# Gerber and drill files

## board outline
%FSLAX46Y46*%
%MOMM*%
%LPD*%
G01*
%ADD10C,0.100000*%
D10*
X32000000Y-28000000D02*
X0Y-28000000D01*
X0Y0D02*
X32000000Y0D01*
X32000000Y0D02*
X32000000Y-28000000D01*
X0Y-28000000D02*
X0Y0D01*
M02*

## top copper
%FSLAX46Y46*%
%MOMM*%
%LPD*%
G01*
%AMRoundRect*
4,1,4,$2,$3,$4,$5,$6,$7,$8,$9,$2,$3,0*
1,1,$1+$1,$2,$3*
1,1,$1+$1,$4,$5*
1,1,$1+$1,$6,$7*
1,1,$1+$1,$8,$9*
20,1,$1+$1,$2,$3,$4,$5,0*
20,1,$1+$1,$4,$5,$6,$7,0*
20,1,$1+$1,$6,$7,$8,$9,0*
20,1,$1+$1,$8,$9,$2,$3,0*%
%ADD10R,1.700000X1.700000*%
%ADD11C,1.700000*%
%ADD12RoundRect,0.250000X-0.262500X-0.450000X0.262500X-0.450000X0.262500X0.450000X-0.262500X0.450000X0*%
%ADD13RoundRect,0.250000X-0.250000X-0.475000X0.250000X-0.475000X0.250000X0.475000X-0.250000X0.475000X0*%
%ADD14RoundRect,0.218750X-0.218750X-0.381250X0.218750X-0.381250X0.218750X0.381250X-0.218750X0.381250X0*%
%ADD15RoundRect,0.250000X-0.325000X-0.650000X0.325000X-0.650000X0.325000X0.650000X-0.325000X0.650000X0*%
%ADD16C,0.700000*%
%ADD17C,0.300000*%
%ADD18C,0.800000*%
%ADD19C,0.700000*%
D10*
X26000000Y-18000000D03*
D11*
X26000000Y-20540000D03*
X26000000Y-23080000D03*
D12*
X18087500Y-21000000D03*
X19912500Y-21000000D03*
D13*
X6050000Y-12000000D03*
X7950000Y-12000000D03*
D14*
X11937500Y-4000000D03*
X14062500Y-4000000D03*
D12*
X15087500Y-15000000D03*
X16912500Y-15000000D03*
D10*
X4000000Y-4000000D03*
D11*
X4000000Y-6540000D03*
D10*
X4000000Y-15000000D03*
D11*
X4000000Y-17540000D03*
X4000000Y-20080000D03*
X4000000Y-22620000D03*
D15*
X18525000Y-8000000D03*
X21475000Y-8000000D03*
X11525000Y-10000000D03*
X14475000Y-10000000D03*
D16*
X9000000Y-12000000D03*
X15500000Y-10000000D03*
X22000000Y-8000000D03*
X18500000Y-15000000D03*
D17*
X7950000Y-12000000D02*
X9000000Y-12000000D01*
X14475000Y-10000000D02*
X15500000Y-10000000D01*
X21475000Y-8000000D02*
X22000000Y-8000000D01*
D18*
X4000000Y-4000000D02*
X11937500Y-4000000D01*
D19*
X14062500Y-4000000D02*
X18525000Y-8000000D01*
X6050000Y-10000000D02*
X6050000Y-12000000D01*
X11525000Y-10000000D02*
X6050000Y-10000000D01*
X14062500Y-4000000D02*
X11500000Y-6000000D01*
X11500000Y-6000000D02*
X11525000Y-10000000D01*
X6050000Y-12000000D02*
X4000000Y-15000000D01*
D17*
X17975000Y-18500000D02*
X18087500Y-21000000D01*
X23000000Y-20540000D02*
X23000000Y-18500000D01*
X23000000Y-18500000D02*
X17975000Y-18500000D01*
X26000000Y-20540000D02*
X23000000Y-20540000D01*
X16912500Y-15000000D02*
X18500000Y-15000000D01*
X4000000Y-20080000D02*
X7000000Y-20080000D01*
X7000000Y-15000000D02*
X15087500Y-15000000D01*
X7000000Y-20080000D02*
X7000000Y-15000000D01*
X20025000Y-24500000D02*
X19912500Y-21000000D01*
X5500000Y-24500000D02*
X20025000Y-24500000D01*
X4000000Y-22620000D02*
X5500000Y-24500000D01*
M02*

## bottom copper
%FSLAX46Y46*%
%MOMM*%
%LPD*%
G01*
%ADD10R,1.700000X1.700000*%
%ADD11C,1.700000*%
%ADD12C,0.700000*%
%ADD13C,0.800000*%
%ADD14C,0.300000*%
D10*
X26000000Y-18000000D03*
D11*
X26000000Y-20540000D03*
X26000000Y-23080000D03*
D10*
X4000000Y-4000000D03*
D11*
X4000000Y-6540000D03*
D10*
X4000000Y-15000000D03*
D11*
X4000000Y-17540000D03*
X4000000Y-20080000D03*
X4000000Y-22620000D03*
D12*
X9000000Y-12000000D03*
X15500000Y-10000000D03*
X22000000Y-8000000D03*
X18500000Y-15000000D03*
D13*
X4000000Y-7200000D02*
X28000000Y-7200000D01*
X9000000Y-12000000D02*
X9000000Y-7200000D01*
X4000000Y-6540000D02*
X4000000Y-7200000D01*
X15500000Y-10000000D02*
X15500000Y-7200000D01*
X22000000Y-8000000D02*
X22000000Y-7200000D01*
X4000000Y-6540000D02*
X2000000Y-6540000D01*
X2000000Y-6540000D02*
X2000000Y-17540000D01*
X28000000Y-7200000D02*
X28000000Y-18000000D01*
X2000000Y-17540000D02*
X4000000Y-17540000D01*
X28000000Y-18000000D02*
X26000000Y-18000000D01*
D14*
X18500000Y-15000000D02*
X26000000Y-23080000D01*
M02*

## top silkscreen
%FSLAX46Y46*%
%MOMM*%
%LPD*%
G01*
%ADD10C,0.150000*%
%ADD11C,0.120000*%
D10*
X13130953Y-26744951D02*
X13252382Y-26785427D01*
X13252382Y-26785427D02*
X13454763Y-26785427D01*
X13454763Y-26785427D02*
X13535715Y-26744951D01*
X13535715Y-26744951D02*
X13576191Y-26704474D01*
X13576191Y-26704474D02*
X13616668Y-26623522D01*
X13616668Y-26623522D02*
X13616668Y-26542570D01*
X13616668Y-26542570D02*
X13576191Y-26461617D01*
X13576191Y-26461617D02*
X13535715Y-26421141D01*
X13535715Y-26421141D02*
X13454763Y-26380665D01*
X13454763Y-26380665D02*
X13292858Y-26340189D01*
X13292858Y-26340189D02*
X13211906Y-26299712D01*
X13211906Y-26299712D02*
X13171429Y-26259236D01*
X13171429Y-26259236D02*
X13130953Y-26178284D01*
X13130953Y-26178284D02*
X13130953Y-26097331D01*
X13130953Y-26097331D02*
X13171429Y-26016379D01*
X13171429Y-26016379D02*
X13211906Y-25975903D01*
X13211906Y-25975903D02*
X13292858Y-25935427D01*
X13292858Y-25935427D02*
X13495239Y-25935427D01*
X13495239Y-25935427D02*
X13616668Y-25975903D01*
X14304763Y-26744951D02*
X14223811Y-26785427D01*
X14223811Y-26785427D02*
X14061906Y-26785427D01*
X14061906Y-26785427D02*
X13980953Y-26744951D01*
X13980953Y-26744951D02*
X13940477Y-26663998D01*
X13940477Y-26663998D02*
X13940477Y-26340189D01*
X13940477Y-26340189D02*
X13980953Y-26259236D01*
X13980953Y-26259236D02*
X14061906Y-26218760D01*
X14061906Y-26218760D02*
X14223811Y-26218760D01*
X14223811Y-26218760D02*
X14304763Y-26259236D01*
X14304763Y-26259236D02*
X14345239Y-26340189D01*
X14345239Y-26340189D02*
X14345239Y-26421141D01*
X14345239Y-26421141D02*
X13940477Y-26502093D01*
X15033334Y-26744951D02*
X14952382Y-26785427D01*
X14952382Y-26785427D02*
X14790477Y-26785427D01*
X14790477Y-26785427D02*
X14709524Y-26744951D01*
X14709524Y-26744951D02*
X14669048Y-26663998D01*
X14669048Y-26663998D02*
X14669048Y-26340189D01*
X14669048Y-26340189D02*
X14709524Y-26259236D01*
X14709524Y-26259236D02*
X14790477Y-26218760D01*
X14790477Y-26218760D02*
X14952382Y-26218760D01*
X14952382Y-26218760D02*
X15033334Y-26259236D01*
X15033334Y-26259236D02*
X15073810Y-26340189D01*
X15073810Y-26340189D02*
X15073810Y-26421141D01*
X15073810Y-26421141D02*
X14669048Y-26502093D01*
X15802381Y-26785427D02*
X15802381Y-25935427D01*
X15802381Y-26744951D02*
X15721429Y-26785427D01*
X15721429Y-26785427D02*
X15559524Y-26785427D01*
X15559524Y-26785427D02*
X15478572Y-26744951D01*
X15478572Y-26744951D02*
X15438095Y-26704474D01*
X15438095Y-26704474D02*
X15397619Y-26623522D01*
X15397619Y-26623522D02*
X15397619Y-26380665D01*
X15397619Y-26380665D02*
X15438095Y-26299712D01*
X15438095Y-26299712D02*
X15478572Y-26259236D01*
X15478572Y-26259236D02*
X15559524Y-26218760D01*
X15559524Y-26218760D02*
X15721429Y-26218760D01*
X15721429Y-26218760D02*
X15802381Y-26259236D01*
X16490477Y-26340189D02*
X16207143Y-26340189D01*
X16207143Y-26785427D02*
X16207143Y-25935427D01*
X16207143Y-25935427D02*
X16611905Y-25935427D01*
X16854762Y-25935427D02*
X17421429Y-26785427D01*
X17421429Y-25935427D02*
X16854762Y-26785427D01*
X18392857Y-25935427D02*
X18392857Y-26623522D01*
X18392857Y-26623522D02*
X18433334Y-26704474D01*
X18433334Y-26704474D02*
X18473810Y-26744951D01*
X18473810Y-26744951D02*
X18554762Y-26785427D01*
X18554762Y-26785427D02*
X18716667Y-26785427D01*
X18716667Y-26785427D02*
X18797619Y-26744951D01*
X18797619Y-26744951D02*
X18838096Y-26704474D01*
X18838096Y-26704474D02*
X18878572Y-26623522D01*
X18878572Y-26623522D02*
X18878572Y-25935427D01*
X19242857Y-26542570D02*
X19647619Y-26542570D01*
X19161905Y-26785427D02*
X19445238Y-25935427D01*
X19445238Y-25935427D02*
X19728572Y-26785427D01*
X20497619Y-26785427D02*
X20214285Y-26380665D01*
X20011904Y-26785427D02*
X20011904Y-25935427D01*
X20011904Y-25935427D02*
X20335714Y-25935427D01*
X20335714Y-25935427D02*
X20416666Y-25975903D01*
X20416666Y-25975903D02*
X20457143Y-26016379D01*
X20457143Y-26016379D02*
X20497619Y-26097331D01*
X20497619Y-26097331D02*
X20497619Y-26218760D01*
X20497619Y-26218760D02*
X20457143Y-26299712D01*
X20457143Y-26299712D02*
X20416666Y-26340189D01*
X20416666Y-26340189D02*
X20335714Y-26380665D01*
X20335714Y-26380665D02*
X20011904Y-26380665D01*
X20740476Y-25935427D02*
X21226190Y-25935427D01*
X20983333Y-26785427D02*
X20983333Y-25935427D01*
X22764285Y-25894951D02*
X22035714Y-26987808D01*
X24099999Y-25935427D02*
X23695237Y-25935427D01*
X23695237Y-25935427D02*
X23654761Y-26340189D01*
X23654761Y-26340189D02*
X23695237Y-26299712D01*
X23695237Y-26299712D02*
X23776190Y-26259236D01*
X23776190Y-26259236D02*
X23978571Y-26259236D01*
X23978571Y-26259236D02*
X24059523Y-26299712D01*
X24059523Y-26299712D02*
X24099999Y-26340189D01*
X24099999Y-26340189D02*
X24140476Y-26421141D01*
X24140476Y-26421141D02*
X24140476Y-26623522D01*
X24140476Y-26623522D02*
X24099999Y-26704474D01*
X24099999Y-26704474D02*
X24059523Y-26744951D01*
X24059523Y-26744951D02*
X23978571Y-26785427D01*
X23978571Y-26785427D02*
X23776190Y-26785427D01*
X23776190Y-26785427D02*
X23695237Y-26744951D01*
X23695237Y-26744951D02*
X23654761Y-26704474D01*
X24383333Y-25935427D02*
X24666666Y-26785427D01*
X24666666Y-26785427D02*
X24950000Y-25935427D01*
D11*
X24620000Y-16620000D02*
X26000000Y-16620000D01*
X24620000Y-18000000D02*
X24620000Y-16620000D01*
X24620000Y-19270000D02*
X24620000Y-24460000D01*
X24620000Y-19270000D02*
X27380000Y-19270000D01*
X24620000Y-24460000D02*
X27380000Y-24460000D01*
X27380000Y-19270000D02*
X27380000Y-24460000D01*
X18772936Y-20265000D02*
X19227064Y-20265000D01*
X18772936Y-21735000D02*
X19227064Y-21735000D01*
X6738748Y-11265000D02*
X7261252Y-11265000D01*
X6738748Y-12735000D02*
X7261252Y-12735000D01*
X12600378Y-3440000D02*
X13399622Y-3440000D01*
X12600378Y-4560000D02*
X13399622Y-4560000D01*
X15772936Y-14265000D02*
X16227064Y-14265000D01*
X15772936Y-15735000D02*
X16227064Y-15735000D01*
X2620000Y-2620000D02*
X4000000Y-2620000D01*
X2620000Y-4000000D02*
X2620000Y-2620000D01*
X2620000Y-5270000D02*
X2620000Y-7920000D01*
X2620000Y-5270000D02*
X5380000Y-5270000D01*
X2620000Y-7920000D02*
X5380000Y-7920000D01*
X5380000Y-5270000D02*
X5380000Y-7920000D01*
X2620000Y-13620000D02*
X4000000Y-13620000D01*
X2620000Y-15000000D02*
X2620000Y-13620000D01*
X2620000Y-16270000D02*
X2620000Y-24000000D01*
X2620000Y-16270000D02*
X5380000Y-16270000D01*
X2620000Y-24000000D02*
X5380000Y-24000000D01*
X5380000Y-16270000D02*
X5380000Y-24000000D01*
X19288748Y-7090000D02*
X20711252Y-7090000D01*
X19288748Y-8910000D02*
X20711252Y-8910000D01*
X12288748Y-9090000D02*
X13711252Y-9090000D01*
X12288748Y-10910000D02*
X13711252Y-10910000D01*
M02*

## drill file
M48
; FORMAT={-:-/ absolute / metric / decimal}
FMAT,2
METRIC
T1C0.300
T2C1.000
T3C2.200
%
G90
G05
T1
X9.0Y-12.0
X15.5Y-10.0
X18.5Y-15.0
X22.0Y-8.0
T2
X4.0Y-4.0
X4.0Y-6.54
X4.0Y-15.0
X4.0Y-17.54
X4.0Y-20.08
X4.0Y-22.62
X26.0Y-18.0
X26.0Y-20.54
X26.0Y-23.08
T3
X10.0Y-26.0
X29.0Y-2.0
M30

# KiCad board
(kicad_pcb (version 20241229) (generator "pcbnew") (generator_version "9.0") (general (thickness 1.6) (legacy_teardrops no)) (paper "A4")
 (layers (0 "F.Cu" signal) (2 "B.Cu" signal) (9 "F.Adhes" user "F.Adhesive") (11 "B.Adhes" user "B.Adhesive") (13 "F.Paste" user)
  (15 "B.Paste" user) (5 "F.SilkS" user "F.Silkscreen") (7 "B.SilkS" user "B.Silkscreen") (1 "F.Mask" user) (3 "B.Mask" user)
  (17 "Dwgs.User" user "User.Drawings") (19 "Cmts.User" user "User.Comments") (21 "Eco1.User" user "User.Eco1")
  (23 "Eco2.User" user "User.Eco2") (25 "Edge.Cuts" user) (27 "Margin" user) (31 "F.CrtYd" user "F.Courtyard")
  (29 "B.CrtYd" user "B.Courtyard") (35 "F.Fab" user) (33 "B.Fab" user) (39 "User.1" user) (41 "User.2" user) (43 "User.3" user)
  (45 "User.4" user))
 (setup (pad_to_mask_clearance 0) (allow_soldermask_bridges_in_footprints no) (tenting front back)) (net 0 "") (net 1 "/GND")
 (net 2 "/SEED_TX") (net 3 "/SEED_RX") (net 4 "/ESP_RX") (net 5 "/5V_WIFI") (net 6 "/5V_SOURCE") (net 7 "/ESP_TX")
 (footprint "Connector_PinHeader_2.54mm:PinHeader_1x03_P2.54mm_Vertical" (layer "F.Cu") (at 26 18)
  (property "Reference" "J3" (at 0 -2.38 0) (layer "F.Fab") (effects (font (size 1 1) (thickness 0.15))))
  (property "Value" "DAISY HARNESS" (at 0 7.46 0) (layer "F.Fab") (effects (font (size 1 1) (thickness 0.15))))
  (fp_line (start -1.38 -1.38) (end 0 -1.38) (stroke (width 0.12) (type solid)) (layer "F.SilkS"))
  (fp_line (start -1.38 0) (end -1.38 -1.38) (stroke (width 0.12) (type solid)) (layer "F.SilkS"))
  (fp_line (start -1.38 1.27) (end -1.38 6.46) (stroke (width 0.12) (type solid)) (layer "F.SilkS"))
  (fp_line (start -1.38 1.27) (end 1.38 1.27) (stroke (width 0.12) (type solid)) (layer "F.SilkS"))
  (fp_line (start -1.38 6.46) (end 1.38 6.46) (stroke (width 0.12) (type solid)) (layer "F.SilkS"))
  (fp_line (start 1.38 1.27) (end 1.38 6.46) (stroke (width 0.12) (type solid)) (layer "F.SilkS"))
  (pad "1" thru_hole rect (at 0 0) (size 1.7 1.7) (drill 1) (layers "*.Cu" "*.Mask") (remove_unused_layers no) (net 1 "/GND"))
  (pad "2" thru_hole circle (at 0 2.54) (size 1.7 1.7) (drill 1) (layers "*.Cu" "*.Mask") (remove_unused_layers no) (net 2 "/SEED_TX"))
  (pad "3" thru_hole circle (at 0 5.08) (size 1.7 1.7) (drill 1) (layers "*.Cu" "*.Mask") (remove_unused_layers no) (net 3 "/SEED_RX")))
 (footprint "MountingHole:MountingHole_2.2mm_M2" (layer "F.Cu") (at 10 26)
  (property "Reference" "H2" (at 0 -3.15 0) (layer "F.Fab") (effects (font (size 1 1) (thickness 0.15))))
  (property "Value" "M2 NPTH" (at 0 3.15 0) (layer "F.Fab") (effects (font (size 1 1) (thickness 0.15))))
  (pad "" np_thru_hole circle (at 0 0) (size 2.2 2.2) (drill 2.2) (layers "*.Cu" "*.Mask")))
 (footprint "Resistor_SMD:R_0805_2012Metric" (layer "F.Cu") (at 19 21)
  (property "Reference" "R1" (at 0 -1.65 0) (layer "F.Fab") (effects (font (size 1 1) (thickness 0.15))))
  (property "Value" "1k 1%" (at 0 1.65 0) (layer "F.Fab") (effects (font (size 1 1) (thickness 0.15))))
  (fp_line (start -0.227064 -0.735) (end 0.227064 -0.735) (stroke (width 0.12) (type solid)) (layer "F.SilkS"))
  (fp_line (start -0.227064 0.735) (end 0.227064 0.735) (stroke (width 0.12) (type solid)) (layer "F.SilkS"))
  (pad "1" smd roundrect (at -0.9125 0) (size 1.025 1.4) (layers "F.Cu" "F.Mask" "F.Paste") (roundrect_rratio 0.243902) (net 2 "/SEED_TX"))
  (pad "2" smd roundrect (at 0.9125 0) (size 1.025 1.4) (layers "F.Cu" "F.Mask" "F.Paste") (roundrect_rratio 0.243902) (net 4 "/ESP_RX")))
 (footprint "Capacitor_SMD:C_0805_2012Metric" (layer "F.Cu") (at 7 12)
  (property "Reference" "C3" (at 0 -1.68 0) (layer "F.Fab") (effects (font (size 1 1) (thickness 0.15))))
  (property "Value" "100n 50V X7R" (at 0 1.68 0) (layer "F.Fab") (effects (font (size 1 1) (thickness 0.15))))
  (fp_line (start -0.261252 -0.735) (end 0.261252 -0.735) (stroke (width 0.12) (type solid)) (layer "F.SilkS"))
  (fp_line (start -0.261252 0.735) (end 0.261252 0.735) (stroke (width 0.12) (type solid)) (layer "F.SilkS"))
  (pad "1" smd roundrect (at -0.95 0) (size 1 1.45) (layers "F.Cu" "F.Mask" "F.Paste") (roundrect_rratio 0.25) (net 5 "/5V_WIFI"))
  (pad "2" smd roundrect (at 0.95 0) (size 1 1.45) (layers "F.Cu" "F.Mask" "F.Paste") (roundrect_rratio 0.25) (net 1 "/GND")))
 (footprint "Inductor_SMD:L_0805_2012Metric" (layer "F.Cu") (at 13 4)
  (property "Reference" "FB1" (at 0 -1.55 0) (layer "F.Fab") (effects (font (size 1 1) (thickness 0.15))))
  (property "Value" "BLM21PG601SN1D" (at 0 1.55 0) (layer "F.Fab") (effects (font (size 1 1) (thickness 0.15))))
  (fp_line (start -0.399622 -0.56) (end 0.399622 -0.56) (stroke (width 0.12) (type solid)) (layer "F.SilkS"))
  (fp_line (start -0.399622 0.56) (end 0.399622 0.56) (stroke (width 0.12) (type solid)) (layer "F.SilkS"))
  (pad "1" smd roundrect (at -1.0625 0) (size 0.875 1.2) (layers "F.Cu" "F.Mask" "F.Paste") (roundrect_rratio 0.25) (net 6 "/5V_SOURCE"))
  (pad "2" smd roundrect (at 1.0625 0) (size 0.875 1.2) (layers "F.Cu" "F.Mask" "F.Paste") (roundrect_rratio 0.25) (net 5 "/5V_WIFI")))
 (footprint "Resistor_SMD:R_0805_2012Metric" (layer "F.Cu") (at 16 15)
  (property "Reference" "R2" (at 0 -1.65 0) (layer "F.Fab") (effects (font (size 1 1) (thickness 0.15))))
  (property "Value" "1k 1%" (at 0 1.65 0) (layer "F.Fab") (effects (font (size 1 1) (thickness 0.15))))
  (fp_line (start -0.227064 -0.735) (end 0.227064 -0.735) (stroke (width 0.12) (type solid)) (layer "F.SilkS"))
  (fp_line (start -0.227064 0.735) (end 0.227064 0.735) (stroke (width 0.12) (type solid)) (layer "F.SilkS"))
  (pad "1" smd roundrect (at -0.9125 0) (size 1.025 1.4) (layers "F.Cu" "F.Mask" "F.Paste") (roundrect_rratio 0.243902) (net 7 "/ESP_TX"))
  (pad "2" smd roundrect (at 0.9125 0) (size 1.025 1.4) (layers "F.Cu" "F.Mask" "F.Paste") (roundrect_rratio 0.243902) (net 3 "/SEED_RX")))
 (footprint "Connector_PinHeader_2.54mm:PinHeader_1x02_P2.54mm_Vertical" (layer "F.Cu") (at 4 4)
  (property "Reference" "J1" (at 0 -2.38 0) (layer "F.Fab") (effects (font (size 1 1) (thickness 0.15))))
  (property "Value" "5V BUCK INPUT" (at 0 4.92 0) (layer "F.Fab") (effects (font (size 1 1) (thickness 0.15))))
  (fp_line (start -1.38 -1.38) (end 0 -1.38) (stroke (width 0.12) (type solid)) (layer "F.SilkS"))
  (fp_line (start -1.38 0) (end -1.38 -1.38) (stroke (width 0.12) (type solid)) (layer "F.SilkS"))
  (fp_line (start -1.38 1.27) (end -1.38 3.92) (stroke (width 0.12) (type solid)) (layer "F.SilkS"))
  (fp_line (start -1.38 1.27) (end 1.38 1.27) (stroke (width 0.12) (type solid)) (layer "F.SilkS"))
  (fp_line (start -1.38 3.92) (end 1.38 3.92) (stroke (width 0.12) (type solid)) (layer "F.SilkS"))
  (fp_line (start 1.38 1.27) (end 1.38 3.92) (stroke (width 0.12) (type solid)) (layer "F.SilkS"))
  (pad "1" thru_hole rect (at 0 0) (size 1.7 1.7) (drill 1) (layers "*.Cu" "*.Mask") (remove_unused_layers no) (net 6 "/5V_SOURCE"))
  (pad "2" thru_hole circle (at 0 2.54) (size 1.7 1.7) (drill 1) (layers "*.Cu" "*.Mask") (remove_unused_layers no) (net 1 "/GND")))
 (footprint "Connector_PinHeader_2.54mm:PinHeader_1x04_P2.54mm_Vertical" (layer "F.Cu") (at 4 15)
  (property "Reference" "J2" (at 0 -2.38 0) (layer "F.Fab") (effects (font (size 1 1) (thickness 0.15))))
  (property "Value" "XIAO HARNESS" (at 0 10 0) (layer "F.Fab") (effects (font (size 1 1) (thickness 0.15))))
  (fp_line (start -1.38 -1.38) (end 0 -1.38) (stroke (width 0.12) (type solid)) (layer "F.SilkS"))
  (fp_line (start -1.38 0) (end -1.38 -1.38) (stroke (width 0.12) (type solid)) (layer "F.SilkS"))
  (fp_line (start -1.38 1.27) (end -1.38 9) (stroke (width 0.12) (type solid)) (layer "F.SilkS"))
  (fp_line (start -1.38 1.27) (end 1.38 1.27) (stroke (width 0.12) (type solid)) (layer "F.SilkS"))
  (fp_line (start -1.38 9) (end 1.38 9) (stroke (width 0.12) (type solid)) (layer "F.SilkS"))
  (fp_line (start 1.38 1.27) (end 1.38 9) (stroke (width 0.12) (type solid)) (layer "F.SilkS"))
  (pad "1" thru_hole rect (at 0 0) (size 1.7 1.7) (drill 1) (layers "*.Cu" "*.Mask") (remove_unused_layers no) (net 5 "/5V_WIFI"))
  (pad "2" thru_hole circle (at 0 2.54) (size 1.7 1.7) (drill 1) (layers "*.Cu" "*.Mask") (remove_unused_layers no) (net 1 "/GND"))
  (pad "3" thru_hole circle (at 0 5.08) (size 1.7 1.7) (drill 1) (layers "*.Cu" "*.Mask") (remove_unused_layers no) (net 7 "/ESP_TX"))
  (pad "4" thru_hole circle (at 0 7.62) (size 1.7 1.7) (drill 1) (layers "*.Cu" "*.Mask") (remove_unused_layers no) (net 4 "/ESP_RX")))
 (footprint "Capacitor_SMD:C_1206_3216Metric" (layer "F.Cu") (at 20 8)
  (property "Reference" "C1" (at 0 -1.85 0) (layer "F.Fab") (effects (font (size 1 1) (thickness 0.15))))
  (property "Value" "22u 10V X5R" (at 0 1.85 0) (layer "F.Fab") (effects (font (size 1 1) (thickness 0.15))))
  (fp_line (start -0.711252 -0.91) (end 0.711252 -0.91) (stroke (width 0.12) (type solid)) (layer "F.SilkS"))
  (fp_line (start -0.711252 0.91) (end 0.711252 0.91) (stroke (width 0.12) (type solid)) (layer "F.SilkS"))
  (pad "1" smd roundrect (at -1.475 0) (size 1.15 1.8) (layers "F.Cu" "F.Mask" "F.Paste") (roundrect_rratio 0.217391) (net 5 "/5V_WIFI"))
  (pad "2" smd roundrect (at 1.475 0) (size 1.15 1.8) (layers "F.Cu" "F.Mask" "F.Paste") (roundrect_rratio 0.217391) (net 1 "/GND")))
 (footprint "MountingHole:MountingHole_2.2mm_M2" (layer "F.Cu") (at 29 2)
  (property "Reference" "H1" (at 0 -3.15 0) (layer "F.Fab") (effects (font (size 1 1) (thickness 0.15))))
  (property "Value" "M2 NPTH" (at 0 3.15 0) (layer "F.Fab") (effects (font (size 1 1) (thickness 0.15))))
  (pad "" np_thru_hole circle (at 0 0) (size 2.2 2.2) (drill 2.2) (layers "*.Cu" "*.Mask")))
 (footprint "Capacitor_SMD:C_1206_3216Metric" (layer "F.Cu") (at 13 10)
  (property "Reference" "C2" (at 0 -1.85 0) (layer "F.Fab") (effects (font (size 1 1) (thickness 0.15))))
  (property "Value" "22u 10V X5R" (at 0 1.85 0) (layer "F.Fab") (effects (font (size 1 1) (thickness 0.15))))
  (fp_line (start -0.711252 -0.91) (end 0.711252 -0.91) (stroke (width 0.12) (type solid)) (layer "F.SilkS"))
  (fp_line (start -0.711252 0.91) (end 0.711252 0.91) (stroke (width 0.12) (type solid)) (layer "F.SilkS"))
  (pad "1" smd roundrect (at -1.475 0) (size 1.15 1.8) (layers "F.Cu" "F.Mask" "F.Paste") (roundrect_rratio 0.217391) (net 5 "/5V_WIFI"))
  (pad "2" smd roundrect (at 1.475 0) (size 1.15 1.8) (layers "F.Cu" "F.Mask" "F.Paste") (roundrect_rratio 0.217391) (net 1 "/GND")))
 (gr_line (start 32 28) (end 0 28) (stroke (width 0.1) (type default)) (layer "Edge.Cuts"))
 (gr_line (start 0 0) (end 32 0) (stroke (width 0.1) (type default)) (layer "Edge.Cuts"))
 (gr_line (start 32 0) (end 32 28) (stroke (width 0.1) (type default)) (layer "Edge.Cuts"))
 (gr_line (start 0 28) (end 0 0) (stroke (width 0.1) (type default)) (layer "Edge.Cuts"))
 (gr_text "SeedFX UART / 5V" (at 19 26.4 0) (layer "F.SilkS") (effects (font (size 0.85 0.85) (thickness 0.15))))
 (segment (start 7.95 12) (end 9 12) (width 0.3) (layer "F.Cu") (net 1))
 (segment (start 14.475 10) (end 15.5 10) (width 0.3) (layer "F.Cu") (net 1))
 (segment (start 21.475 8) (end 22 8) (width 0.3) (layer "F.Cu") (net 1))
 (via (at 9 12) (size 0.7) (drill 0.3) (layers "F.Cu" "B.Cu") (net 1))
 (via (at 15.5 10) (size 0.7) (drill 0.3) (layers "F.Cu" "B.Cu") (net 1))
 (via (at 22 8) (size 0.7) (drill 0.3) (layers "F.Cu" "B.Cu") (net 1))
 (segment (start 4 7.2) (end 28 7.2) (width 0.8) (layer "B.Cu") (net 1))
 (segment (start 9 12) (end 9 7.2) (width 0.8) (layer "B.Cu") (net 1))
 (segment (start 4 6.54) (end 4 7.2) (width 0.8) (layer "B.Cu") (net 1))
 (segment (start 15.5 10) (end 15.5 7.2) (width 0.8) (layer "B.Cu") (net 1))
 (segment (start 22 8) (end 22 7.2) (width 0.8) (layer "B.Cu") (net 1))
 (segment (start 4 6.54) (end 2 6.54) (width 0.8) (layer "B.Cu") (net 1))
 (segment (start 2 6.54) (end 2 17.54) (width 0.8) (layer "B.Cu") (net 1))
 (segment (start 28 7.2) (end 28 18) (width 0.8) (layer "B.Cu") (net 1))
 (segment (start 2 17.54) (end 4 17.54) (width 0.8) (layer "B.Cu") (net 1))
 (segment (start 28 18) (end 26 18) (width 0.8) (layer "B.Cu") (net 1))
 (segment (start 4 4) (end 11.9375 4) (width 0.8) (layer "F.Cu") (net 6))
 (segment (start 14.0625 4) (end 18.525 8) (width 0.7) (layer "F.Cu") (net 5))
 (segment (start 6.05 10) (end 6.05 12) (width 0.7) (layer "F.Cu") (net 5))
 (segment (start 11.525 10) (end 6.05 10) (width 0.7) (layer "F.Cu") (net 5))
 (segment (start 14.0625 4) (end 11.5 6) (width 0.7) (layer "F.Cu") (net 5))
 (segment (start 11.5 6) (end 11.525 10) (width 0.7) (layer "F.Cu") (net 5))
 (segment (start 6.05 12) (end 4 15) (width 0.7) (layer "F.Cu") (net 5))
 (segment (start 17.975 18.5) (end 18.0875 21) (width 0.3) (layer "F.Cu") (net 2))
 (segment (start 23 20.54) (end 23 18.5) (width 0.3) (layer "F.Cu") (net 2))
 (segment (start 23 18.5) (end 17.975 18.5) (width 0.3) (layer "F.Cu") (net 2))
 (segment (start 26 20.54) (end 23 20.54) (width 0.3) (layer "F.Cu") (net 2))
 (segment (start 16.9125 15) (end 18.5 15) (width 0.3) (layer "F.Cu") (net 3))
 (via (at 18.5 15) (size 0.7) (drill 0.3) (layers "F.Cu" "B.Cu") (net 3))
 (segment (start 18.5 15) (end 26 23.08) (width 0.3) (layer "B.Cu") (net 3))
 (segment (start 4 20.08) (end 7 20.08) (width 0.3) (layer "F.Cu") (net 7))
 (segment (start 7 15) (end 15.0875 15) (width 0.3) (layer "F.Cu") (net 7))
 (segment (start 7 20.08) (end 7 15) (width 0.3) (layer "F.Cu") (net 7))
 (segment (start 20.025 24.5) (end 19.9125 21) (width 0.3) (layer "F.Cu") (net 4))
 (segment (start 5.5 24.5) (end 20.025 24.5) (width 0.3) (layer "F.Cu") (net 4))
 (segment (start 4 22.62) (end 5.5 24.5) (width 0.3) (layer "F.Cu") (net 4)))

